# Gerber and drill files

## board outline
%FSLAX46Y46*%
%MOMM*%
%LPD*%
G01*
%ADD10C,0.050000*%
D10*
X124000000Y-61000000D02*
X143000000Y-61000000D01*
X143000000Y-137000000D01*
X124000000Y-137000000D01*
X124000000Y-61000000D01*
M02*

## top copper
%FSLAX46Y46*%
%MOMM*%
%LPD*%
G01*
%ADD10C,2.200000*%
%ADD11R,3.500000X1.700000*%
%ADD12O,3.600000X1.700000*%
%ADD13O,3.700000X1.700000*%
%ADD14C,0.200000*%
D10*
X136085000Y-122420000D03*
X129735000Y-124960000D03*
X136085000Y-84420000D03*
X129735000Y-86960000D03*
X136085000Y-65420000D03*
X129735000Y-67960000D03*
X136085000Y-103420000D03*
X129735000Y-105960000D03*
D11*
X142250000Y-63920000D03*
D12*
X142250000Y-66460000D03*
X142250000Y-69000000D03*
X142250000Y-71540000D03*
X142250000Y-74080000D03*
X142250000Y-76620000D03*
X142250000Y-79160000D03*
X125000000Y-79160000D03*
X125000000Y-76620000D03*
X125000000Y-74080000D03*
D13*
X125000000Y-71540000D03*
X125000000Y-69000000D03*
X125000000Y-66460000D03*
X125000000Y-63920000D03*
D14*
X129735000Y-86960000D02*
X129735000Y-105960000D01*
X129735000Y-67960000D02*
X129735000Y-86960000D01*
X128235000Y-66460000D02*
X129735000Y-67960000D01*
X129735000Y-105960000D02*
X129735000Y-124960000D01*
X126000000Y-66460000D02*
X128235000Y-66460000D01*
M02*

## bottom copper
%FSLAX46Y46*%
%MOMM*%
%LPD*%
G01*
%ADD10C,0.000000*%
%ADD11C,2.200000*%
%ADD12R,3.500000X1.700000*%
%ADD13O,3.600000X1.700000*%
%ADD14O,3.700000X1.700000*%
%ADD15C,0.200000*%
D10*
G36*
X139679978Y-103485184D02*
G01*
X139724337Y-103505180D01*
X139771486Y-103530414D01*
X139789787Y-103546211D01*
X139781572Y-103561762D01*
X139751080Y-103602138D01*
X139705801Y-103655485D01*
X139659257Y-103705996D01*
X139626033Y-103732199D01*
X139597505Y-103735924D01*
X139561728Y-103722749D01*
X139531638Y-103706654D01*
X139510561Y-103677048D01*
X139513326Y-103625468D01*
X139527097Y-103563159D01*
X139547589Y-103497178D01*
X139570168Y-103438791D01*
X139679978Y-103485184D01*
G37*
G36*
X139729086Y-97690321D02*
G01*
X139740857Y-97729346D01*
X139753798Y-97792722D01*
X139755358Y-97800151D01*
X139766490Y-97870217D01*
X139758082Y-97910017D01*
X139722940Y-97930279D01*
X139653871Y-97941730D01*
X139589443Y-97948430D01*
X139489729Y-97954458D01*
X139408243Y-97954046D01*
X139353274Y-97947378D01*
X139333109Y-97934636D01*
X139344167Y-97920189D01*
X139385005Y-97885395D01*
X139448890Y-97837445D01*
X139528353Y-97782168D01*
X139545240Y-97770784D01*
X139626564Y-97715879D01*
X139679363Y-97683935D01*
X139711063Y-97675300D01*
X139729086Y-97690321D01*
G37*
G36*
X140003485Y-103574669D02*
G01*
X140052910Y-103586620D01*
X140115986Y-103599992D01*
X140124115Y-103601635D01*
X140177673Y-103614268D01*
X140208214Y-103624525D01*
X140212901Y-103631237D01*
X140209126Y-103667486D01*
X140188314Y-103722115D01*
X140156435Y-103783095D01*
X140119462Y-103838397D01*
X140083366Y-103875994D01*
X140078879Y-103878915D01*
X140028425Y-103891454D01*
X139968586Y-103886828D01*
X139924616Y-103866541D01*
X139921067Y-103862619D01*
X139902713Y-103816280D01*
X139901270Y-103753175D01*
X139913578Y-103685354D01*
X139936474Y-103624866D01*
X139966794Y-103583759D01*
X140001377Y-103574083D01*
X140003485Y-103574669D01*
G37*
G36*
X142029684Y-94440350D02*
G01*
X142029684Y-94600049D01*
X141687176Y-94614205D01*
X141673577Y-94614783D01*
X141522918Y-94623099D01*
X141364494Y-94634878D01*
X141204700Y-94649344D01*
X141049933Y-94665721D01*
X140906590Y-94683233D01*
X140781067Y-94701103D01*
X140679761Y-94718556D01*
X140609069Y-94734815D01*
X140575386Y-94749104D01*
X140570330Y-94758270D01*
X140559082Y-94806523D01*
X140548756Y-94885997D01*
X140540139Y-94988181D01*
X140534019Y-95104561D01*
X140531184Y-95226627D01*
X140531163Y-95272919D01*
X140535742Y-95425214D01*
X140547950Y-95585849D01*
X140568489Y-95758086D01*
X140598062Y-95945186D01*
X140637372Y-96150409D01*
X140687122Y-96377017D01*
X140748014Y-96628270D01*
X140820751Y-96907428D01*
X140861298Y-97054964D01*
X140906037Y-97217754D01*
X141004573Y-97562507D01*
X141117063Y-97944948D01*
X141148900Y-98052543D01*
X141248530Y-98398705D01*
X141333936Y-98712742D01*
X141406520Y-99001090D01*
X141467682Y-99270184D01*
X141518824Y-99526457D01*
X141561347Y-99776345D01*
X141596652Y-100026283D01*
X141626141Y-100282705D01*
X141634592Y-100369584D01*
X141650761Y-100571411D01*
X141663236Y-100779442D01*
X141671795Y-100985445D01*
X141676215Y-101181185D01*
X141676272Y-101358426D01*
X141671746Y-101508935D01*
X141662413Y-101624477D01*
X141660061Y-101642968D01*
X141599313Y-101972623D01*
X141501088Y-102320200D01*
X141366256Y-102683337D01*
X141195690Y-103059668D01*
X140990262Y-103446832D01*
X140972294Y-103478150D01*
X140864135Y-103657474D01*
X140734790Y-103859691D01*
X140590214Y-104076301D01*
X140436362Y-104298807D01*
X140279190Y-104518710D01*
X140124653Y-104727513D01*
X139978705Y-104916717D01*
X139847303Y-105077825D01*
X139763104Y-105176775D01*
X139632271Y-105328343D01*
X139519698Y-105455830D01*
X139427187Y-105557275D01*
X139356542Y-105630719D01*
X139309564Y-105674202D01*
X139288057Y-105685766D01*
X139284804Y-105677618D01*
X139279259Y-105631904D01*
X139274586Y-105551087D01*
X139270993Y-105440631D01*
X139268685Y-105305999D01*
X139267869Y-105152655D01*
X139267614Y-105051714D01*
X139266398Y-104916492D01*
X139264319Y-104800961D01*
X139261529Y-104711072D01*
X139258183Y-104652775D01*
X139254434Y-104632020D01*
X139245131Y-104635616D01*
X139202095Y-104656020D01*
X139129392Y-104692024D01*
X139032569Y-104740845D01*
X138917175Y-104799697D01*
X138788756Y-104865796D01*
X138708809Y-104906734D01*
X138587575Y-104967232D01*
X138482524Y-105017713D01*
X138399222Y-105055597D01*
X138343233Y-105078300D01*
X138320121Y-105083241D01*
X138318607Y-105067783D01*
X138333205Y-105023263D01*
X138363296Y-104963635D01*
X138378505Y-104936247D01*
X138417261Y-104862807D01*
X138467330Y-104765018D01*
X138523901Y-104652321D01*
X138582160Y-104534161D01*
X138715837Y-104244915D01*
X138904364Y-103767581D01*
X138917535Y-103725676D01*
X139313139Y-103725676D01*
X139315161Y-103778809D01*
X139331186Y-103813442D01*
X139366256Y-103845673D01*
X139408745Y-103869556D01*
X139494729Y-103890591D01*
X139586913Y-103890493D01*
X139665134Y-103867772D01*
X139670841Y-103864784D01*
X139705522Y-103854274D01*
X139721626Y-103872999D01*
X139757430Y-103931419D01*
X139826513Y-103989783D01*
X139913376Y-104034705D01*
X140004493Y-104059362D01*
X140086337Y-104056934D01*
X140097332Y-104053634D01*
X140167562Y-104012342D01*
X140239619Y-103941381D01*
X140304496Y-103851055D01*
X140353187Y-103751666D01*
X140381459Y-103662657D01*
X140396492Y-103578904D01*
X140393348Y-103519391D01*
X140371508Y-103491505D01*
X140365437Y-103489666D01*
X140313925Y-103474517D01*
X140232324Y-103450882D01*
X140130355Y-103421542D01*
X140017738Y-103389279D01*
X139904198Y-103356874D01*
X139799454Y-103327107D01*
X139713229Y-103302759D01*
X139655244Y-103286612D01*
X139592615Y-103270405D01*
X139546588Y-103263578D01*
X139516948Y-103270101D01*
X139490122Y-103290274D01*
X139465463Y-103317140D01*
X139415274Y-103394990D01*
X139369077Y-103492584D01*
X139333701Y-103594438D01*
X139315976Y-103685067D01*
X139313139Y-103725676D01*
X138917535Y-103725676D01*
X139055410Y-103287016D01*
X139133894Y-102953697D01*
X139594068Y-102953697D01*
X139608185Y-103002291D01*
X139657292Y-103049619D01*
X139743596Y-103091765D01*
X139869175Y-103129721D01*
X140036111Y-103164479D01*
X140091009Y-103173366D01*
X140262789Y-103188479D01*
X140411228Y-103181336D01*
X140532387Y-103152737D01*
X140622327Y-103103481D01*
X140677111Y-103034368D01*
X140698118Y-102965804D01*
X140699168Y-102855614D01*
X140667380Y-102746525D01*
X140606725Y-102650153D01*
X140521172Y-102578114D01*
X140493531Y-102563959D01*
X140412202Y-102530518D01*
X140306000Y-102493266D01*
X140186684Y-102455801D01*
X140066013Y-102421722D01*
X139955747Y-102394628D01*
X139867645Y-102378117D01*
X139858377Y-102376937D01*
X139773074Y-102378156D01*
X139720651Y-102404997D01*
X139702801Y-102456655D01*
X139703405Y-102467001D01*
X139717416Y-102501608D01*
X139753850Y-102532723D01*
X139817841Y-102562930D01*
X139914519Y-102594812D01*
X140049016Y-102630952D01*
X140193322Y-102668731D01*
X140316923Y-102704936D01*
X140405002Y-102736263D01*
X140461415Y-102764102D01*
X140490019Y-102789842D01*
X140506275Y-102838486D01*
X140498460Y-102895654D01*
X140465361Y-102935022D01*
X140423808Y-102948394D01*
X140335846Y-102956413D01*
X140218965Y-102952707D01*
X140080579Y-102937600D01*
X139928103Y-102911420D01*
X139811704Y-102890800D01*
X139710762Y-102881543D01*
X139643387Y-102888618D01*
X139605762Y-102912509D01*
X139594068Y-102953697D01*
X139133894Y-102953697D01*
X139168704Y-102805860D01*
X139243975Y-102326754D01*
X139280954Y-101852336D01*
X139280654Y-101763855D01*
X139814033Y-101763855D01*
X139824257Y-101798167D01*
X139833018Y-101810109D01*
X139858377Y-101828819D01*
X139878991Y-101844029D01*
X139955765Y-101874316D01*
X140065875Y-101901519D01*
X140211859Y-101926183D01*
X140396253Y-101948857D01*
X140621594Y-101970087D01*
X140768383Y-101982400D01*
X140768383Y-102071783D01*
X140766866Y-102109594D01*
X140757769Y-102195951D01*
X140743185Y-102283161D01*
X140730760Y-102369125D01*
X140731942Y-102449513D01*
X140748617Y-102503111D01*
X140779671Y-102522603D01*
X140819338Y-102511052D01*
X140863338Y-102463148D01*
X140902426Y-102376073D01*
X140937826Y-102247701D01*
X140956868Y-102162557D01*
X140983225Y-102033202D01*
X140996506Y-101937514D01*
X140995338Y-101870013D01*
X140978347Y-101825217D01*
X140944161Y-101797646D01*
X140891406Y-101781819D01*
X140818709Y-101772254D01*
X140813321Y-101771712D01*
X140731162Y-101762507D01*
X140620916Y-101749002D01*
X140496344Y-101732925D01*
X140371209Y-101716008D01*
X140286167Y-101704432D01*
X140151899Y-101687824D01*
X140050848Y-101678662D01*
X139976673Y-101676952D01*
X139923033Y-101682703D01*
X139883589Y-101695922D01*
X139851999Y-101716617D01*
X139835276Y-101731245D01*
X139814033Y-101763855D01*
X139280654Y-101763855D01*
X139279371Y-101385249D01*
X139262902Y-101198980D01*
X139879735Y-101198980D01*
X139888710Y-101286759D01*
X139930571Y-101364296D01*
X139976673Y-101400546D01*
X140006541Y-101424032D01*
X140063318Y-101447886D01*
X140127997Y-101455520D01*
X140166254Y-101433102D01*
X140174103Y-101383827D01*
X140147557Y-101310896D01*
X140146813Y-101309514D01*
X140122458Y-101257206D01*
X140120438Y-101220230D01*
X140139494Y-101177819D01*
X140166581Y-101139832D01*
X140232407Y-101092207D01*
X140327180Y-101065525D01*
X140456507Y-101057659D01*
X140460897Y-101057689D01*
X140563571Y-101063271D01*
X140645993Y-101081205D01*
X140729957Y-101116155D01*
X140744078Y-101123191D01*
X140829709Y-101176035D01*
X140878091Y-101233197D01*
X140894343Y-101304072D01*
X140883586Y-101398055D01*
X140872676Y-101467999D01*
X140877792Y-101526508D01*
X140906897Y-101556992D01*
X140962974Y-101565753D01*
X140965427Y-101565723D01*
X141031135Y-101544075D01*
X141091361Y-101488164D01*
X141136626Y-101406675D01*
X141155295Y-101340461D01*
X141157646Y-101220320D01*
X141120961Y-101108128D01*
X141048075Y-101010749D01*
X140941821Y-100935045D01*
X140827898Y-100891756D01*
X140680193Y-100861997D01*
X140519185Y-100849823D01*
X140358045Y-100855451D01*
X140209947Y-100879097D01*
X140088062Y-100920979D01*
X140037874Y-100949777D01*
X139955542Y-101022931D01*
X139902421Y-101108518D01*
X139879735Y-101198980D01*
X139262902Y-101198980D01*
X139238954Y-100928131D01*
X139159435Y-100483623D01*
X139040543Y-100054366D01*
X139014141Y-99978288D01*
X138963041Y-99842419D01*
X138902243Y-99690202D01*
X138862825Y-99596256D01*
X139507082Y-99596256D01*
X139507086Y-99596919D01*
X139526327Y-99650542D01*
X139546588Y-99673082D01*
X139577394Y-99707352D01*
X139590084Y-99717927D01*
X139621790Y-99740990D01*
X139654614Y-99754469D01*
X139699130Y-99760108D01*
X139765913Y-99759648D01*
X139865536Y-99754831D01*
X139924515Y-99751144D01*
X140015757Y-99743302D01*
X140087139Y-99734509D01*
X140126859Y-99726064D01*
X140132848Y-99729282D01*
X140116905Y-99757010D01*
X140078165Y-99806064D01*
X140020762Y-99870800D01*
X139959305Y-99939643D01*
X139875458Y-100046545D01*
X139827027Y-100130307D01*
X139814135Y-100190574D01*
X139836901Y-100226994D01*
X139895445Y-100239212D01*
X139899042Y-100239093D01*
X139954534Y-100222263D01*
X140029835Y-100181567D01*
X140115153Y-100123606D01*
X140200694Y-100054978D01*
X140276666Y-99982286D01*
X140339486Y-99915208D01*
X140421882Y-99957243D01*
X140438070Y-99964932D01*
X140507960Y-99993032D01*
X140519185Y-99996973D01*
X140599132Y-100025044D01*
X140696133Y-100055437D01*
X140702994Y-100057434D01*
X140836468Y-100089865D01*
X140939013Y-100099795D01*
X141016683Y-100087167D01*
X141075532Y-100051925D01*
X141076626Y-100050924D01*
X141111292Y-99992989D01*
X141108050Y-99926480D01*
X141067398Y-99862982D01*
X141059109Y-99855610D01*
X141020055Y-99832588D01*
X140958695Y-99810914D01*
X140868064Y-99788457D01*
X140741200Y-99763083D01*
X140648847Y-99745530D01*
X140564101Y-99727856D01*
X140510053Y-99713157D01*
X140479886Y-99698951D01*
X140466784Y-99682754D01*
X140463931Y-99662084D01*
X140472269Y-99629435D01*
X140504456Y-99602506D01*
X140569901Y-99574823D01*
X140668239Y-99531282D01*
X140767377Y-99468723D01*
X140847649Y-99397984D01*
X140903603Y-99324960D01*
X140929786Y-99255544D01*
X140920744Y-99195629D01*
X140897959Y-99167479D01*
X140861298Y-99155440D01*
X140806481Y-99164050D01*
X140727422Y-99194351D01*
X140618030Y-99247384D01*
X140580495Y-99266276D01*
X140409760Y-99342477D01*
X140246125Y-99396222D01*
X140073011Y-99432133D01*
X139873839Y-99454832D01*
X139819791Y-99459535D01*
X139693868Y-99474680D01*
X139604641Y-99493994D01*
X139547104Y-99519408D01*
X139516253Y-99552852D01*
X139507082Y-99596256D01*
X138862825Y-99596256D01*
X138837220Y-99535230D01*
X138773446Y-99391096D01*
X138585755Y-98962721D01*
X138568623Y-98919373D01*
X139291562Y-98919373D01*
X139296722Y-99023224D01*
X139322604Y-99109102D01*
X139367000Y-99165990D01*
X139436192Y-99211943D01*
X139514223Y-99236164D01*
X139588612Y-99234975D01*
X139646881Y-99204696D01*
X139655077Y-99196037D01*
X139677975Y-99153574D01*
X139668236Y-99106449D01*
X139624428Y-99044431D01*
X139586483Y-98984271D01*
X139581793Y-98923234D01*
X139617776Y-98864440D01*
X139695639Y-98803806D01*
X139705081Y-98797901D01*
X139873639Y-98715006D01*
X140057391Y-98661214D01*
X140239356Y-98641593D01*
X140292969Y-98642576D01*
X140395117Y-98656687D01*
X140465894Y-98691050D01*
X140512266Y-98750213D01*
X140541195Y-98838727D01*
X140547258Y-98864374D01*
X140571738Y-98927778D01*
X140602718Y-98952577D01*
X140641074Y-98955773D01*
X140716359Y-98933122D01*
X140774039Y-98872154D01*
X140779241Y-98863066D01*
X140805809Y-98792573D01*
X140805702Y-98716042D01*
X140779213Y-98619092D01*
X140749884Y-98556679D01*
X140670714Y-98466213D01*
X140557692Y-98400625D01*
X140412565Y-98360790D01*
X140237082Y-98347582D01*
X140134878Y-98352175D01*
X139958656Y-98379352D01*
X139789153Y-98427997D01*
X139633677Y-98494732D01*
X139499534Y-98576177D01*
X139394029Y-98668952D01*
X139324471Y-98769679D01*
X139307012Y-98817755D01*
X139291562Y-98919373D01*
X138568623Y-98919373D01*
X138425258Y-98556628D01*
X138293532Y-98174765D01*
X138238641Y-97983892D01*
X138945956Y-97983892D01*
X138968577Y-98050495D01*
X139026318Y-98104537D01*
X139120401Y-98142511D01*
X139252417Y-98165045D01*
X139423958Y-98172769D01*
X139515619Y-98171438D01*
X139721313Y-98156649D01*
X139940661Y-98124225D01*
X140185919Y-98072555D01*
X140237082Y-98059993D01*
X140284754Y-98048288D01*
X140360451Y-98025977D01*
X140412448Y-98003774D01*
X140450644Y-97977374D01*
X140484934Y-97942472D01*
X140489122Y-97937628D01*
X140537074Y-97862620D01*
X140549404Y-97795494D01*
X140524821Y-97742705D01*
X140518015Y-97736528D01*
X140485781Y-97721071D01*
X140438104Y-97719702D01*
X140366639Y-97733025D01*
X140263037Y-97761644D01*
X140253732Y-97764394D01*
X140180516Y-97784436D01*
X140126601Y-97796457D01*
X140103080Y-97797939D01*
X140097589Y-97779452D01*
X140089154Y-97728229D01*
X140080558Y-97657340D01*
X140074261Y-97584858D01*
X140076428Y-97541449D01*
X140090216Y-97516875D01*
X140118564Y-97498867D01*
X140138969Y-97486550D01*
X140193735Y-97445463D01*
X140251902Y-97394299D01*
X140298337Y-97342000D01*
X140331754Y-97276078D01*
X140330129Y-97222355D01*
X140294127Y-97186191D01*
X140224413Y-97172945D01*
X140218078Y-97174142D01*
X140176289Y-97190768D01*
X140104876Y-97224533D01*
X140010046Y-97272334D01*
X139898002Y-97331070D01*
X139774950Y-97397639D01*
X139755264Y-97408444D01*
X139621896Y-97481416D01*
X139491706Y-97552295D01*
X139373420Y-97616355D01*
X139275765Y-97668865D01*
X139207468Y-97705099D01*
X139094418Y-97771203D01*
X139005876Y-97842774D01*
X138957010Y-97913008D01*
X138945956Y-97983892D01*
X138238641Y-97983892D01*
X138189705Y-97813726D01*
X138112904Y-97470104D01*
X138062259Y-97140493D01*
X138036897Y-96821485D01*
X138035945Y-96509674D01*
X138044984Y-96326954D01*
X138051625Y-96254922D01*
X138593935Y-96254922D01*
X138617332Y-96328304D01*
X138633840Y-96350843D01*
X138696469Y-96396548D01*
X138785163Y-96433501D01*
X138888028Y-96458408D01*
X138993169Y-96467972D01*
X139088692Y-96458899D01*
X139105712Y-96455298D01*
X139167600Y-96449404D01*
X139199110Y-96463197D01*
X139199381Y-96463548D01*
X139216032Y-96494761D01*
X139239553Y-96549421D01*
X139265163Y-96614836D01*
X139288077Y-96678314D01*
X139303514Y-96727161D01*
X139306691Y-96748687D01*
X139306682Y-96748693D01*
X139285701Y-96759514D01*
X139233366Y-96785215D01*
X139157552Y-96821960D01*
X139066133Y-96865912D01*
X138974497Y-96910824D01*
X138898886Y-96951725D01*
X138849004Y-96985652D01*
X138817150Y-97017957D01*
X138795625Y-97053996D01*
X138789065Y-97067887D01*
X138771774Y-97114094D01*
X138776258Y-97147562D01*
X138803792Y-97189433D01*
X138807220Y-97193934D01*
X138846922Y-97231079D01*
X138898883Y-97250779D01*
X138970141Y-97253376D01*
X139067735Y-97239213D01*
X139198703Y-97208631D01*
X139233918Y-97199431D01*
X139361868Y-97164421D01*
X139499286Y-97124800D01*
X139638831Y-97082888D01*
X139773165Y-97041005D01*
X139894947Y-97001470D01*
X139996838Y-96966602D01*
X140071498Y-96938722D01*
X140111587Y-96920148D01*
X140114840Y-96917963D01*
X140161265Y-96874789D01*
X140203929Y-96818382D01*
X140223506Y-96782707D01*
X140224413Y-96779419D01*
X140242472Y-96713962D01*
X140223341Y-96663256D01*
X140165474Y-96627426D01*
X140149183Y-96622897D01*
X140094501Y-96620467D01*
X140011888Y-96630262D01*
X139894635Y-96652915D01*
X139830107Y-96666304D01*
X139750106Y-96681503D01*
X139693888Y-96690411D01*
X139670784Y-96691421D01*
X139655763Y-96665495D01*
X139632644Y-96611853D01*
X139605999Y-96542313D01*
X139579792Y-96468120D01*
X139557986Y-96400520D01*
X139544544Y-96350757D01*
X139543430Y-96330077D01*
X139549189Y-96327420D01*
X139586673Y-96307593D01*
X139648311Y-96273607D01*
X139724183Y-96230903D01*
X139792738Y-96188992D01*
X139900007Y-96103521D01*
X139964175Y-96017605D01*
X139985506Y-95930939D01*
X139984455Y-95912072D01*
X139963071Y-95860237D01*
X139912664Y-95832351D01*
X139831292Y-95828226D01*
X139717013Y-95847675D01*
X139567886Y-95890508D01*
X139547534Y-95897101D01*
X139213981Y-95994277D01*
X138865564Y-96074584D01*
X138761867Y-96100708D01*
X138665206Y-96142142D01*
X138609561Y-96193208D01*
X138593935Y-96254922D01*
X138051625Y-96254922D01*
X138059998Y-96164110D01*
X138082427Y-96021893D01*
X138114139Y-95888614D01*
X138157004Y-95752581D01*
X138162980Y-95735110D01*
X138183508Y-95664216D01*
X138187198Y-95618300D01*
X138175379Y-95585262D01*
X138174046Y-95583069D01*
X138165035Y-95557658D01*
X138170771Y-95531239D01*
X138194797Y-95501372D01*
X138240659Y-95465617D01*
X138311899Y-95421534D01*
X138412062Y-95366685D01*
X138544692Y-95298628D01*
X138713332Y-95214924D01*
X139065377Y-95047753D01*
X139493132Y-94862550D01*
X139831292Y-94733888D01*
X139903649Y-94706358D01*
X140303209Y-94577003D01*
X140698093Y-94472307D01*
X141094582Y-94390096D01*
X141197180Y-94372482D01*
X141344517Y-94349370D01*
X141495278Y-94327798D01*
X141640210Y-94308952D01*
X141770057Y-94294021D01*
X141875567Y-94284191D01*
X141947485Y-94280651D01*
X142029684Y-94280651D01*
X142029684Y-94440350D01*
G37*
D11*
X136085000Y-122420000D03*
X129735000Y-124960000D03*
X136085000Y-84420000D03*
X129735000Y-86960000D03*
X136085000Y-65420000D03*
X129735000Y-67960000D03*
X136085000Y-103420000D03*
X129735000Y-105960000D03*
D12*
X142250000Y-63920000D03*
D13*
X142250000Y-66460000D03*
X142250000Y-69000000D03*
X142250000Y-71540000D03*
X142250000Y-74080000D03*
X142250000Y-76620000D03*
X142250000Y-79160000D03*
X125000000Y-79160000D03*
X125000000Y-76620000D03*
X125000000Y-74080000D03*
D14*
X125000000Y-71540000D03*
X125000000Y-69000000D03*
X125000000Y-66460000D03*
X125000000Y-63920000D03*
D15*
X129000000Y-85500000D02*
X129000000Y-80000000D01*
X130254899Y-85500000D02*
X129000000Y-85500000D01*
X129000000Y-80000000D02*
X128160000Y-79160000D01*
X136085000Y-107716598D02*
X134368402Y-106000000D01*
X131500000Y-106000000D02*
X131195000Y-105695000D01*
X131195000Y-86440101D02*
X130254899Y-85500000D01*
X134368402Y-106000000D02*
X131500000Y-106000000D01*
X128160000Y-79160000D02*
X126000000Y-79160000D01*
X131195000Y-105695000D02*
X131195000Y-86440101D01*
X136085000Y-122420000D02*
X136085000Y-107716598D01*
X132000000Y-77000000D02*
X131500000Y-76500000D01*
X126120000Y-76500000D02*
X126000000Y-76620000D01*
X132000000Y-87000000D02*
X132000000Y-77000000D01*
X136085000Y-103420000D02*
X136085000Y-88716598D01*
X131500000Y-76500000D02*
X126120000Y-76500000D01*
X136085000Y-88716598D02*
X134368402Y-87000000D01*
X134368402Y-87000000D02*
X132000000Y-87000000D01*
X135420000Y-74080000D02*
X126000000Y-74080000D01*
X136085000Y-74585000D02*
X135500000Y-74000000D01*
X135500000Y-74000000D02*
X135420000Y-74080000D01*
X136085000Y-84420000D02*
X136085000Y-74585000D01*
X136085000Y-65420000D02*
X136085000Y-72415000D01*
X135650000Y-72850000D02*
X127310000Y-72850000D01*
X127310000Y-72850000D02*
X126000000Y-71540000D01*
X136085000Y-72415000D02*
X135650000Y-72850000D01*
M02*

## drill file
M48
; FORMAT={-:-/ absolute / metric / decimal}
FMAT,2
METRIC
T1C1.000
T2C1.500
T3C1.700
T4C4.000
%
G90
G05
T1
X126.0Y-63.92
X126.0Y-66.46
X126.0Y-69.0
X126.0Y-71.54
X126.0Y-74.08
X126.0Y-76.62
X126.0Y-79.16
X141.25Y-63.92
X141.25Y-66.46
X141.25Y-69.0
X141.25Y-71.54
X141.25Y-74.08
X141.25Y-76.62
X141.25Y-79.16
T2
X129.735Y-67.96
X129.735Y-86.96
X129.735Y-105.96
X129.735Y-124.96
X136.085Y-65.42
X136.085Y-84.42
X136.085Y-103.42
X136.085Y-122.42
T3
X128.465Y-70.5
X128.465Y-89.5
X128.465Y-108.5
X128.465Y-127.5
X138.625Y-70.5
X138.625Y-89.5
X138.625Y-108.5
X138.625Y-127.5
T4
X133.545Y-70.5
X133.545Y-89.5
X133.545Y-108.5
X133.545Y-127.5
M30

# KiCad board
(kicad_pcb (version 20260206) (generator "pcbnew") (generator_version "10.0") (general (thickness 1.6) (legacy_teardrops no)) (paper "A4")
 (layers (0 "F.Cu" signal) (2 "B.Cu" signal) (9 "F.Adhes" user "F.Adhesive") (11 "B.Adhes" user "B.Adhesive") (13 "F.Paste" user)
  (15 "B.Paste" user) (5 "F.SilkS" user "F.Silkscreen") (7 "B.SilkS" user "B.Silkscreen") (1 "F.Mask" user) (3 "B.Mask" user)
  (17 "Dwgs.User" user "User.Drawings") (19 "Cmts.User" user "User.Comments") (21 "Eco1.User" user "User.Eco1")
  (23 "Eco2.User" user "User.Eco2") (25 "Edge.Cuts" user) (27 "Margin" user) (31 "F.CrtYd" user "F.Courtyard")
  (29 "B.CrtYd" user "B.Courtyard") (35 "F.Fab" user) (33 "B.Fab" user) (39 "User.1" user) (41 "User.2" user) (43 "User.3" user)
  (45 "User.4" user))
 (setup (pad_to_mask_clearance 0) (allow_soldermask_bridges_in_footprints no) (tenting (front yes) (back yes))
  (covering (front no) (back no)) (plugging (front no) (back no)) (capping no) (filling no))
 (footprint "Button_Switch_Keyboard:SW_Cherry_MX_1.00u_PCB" (layer "F.Cu") (at 136.085 122.42)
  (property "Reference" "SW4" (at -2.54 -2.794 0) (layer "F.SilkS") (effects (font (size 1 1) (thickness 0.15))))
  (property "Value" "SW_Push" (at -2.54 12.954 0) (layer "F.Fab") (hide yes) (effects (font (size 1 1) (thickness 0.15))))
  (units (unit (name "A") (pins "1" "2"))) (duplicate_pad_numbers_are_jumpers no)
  (pad "" np_thru_hole circle (at -7.62 5.08) (size 1.7 1.7) (drill 1.7) (layers "*.Cu" "*.Mask"))
  (pad "" np_thru_hole circle (at -2.54 5.08) (size 4 4) (drill 4) (layers "*.Cu" "*.Mask"))
  (pad "" np_thru_hole circle (at 2.54 5.08) (size 1.7 1.7) (drill 1.7) (layers "*.Cu" "*.Mask"))
  (pad "1" thru_hole circle (at 0 0) (size 2.2 2.2) (drill 1.5) (layers "*.Cu" "*.Mask") (remove_unused_layers no)
   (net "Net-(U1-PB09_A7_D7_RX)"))
  (pad "2" thru_hole circle (at -6.35 2.54) (size 2.2 2.2) (drill 1.5) (layers "*.Cu" "*.Mask") (remove_unused_layers no) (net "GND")))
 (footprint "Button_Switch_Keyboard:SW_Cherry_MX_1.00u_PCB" (layer "F.Cu") (at 136.085 84.42)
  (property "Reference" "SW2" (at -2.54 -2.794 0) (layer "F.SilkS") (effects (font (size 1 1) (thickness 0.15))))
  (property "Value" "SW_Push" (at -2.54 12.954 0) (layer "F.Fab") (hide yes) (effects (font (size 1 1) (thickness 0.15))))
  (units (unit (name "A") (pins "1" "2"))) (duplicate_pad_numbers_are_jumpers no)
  (pad "" np_thru_hole circle (at -7.62 5.08) (size 1.7 1.7) (drill 1.7) (layers "*.Cu" "*.Mask"))
  (pad "" np_thru_hole circle (at -2.54 5.08) (size 4 4) (drill 4) (layers "*.Cu" "*.Mask"))
  (pad "" np_thru_hole circle (at 2.54 5.08) (size 1.7 1.7) (drill 1.7) (layers "*.Cu" "*.Mask"))
  (pad "1" thru_hole circle (at 0 0) (size 2.2 2.2) (drill 1.5) (layers "*.Cu" "*.Mask") (remove_unused_layers no)
   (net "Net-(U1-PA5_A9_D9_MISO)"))
  (pad "2" thru_hole circle (at -6.35 2.54) (size 2.2 2.2) (drill 1.5) (layers "*.Cu" "*.Mask") (remove_unused_layers no) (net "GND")))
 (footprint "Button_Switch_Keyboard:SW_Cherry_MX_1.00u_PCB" (layer "F.Cu") (at 136.085 65.42)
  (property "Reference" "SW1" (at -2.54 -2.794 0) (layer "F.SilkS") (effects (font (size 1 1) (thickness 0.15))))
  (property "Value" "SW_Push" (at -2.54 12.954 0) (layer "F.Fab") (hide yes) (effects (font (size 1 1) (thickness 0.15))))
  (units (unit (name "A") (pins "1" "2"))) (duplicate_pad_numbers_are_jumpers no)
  (pad "" np_thru_hole circle (at -7.62 5.08) (size 1.7 1.7) (drill 1.7) (layers "*.Cu" "*.Mask"))
  (pad "" np_thru_hole circle (at -2.54 5.08) (size 4 4) (drill 4) (layers "*.Cu" "*.Mask"))
  (pad "" np_thru_hole circle (at 2.54 5.08) (size 1.7 1.7) (drill 1.7) (layers "*.Cu" "*.Mask"))
  (pad "1" thru_hole circle (at 0 0) (size 2.2 2.2) (drill 1.5) (layers "*.Cu" "*.Mask") (remove_unused_layers no)
   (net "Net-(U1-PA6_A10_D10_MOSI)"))
  (pad "2" thru_hole circle (at -6.35 2.54) (size 2.2 2.2) (drill 1.5) (layers "*.Cu" "*.Mask") (remove_unused_layers no) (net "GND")))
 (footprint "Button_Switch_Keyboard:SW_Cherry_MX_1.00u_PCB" (layer "F.Cu") (at 136.085 103.42)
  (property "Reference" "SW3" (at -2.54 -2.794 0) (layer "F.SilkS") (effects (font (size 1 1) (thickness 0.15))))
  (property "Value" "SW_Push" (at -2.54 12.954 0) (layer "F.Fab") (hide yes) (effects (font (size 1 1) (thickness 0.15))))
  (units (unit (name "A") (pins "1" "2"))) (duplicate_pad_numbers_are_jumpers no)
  (pad "" np_thru_hole circle (at -7.62 5.08) (size 1.7 1.7) (drill 1.7) (layers "*.Cu" "*.Mask"))
  (pad "" np_thru_hole circle (at -2.54 5.08) (size 4 4) (drill 4) (layers "*.Cu" "*.Mask"))
  (pad "" np_thru_hole circle (at 2.54 5.08) (size 1.7 1.7) (drill 1.7) (layers "*.Cu" "*.Mask"))
  (pad "1" thru_hole circle (at 0 0) (size 2.2 2.2) (drill 1.5) (layers "*.Cu" "*.Mask") (remove_unused_layers no)
   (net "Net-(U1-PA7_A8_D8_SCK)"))
  (pad "2" thru_hole circle (at -6.35 2.54) (size 2.2 2.2) (drill 1.5) (layers "*.Cu" "*.Mask") (remove_unused_layers no) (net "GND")))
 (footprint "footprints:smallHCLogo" (layer "B.Cu") (at 140.029 100 -90)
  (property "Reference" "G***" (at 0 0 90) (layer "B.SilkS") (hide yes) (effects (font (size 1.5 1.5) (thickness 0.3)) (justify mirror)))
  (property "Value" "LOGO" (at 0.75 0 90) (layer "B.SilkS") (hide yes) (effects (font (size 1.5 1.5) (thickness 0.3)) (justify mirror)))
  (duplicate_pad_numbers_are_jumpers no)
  (fp_poly
   (pts (xy 3.706654 0.497362) (xy 3.722749 0.467272) (xy 3.735924 0.431495) (xy 3.732199 0.402967) (xy 3.705996 0.369743)
    (xy 3.655485 0.323199) (xy 3.602138 0.27792) (xy 3.561762 0.247428) (xy 3.546211 0.239213) (xy 3.530414 0.257514) (xy 3.50518 0.304663)
    (xy 3.485184 0.349022) (xy 3.438791 0.458832) (xy 3.497178 0.481411) (xy 3.563159 0.501903) (xy 3.625468 0.515674)
    (xy 3.677048 0.518439))
   (stroke (width 0) (type solid)) (fill yes) (layer "B.Cu"))
  (fp_poly
   (pts (xy -2.052622 0.675726) (xy -2.045954 0.620757) (xy -2.045542 0.539271) (xy -2.05157 0.439557) (xy -2.05827 0.375129)
    (xy -2.069721 0.30606) (xy -2.089983 0.270918) (xy -2.129783 0.26251) (xy -2.199849 0.273642) (xy -2.207278 0.275202)
    (xy -2.270654 0.288143) (xy -2.309679 0.299914) (xy -2.3247 0.317937) (xy -2.316065 0.349637) (xy -2.284121 0.402436)
    (xy -2.229216 0.48376) (xy -2.217832 0.500647) (xy -2.162555 0.58011) (xy -2.114605 0.643995) (xy -2.079811 0.684833)
    (xy -2.065364 0.695891))
   (stroke (width 0) (type solid)) (fill yes) (layer "B.Cu"))
  (fp_poly
   (pts (xy 3.81628 0.126287) (xy 3.862619 0.107933) (xy 3.866541 0.104384) (xy 3.886828 0.060414) (xy 3.891454 0.000575)
    (xy 3.878915 -0.049879) (xy 3.875994 -0.054366) (xy 3.838397 -0.090462) (xy 3.783095 -0.127435) (xy 3.722115 -0.159314)
    (xy 3.667486 -0.180126) (xy 3.631237 -0.183901) (xy 3.624525 -0.179214) (xy 3.614268 -0.148673) (xy 3.601635 -0.095115)
    (xy 3.599992 -0.086986) (xy 3.58662 -0.02391) (xy 3.574669 0.025515) (xy 3.574083 0.027623) (xy 3.583759 0.062206)
    (xy 3.624866 0.092526) (xy 3.685354 0.115422) (xy 3.753175 0.12773))
   (stroke (width 0) (type solid)) (fill yes) (layer "B.Cu"))
  (fp_poly
   (pts (xy -3.178515 1.992103) (xy -2.859507 1.966741) (xy -2.529896 1.916096) (xy -2.186274 1.839295) (xy -1.825235 1.735468)
    (xy -1.443372 1.603742) (xy -1.037279 1.443245) (xy -0.608904 1.255554) (xy -0.46477 1.19178) (xy -0.309798 1.126757)
    (xy -0.157581 1.065959) (xy -0.021712 1.014859) (xy 0.054366 0.988457) (xy 0.483623 0.869565) (xy 0.928131 0.790046)
    (xy 1.385249 0.749629) (xy 1.852336 0.748046) (xy 2.326754 0.785025) (xy 2.80586 0.860296) (xy 3.287016 0.97359) (xy 3.767581 1.124636)
    (xy 4.244915 1.313163) (xy 4.534161 1.44684) (xy 4.652321 1.505099) (xy 4.765018 1.56167) (xy 4.862807 1.611739) (xy 4.936247 1.650495)
    (xy 4.963635 1.665704) (xy 5.023263 1.695795) (xy 5.067783 1.710393) (xy 5.083241 1.708879) (xy 5.0783 1.685767) (xy 5.055597 1.629778)
    (xy 5.017713 1.546476) (xy 4.967232 1.441425) (xy 4.906734 1.320191) (xy 4.865796 1.240244) (xy 4.799697 1.111825)
    (xy 4.740845 0.996431) (xy 4.692024 0.899608) (xy 4.65602 0.826905) (xy 4.635616 0.783869) (xy 4.63202 0.774566) (xy 4.652775 0.770817)
    (xy 4.711072 0.767471) (xy 4.800961 0.764681) (xy 4.916492 0.762602) (xy 5.051714 0.761386) (xy 5.152655 0.761131)
    (xy 5.305999 0.760315) (xy 5.440631 0.758007) (xy 5.551087 0.754414) (xy 5.631904 0.749741) (xy 5.677618 0.744196)
    (xy 5.685766 0.740943) (xy 5.674202 0.719436) (xy 5.630719 0.672458) (xy 5.557275 0.601813) (xy 5.45583 0.509302) (xy 5.328343 0.396729)
    (xy 5.176775 0.265896) (xy 5.077825 0.181697) (xy 4.916717 0.050295) (xy 4.727513 -0.095653) (xy 4.51871 -0.25019)
    (xy 4.298807 -0.407362) (xy 4.076301 -0.561214) (xy 3.859691 -0.70579) (xy 3.657474 -0.835135) (xy 3.47815 -0.943294)
    (xy 3.446832 -0.961262) (xy 3.059668 -1.16669) (xy 2.683337 -1.337256) (xy 2.3202 -1.472088) (xy 1.972623 -1.570313)
    (xy 1.642968 -1.631061) (xy 1.624477 -1.633413) (xy 1.508935 -1.642746) (xy 1.358426 -1.647272) (xy 1.181185 -1.647215)
    (xy 0.985445 -1.642795) (xy 0.779442 -1.634236) (xy 0.571411 -1.621761) (xy 0.369584 -1.605592) (xy 0.282705 -1.597141)
    (xy 0.026283 -1.567652) (xy -0.223655 -1.532347) (xy -0.473543 -1.489824) (xy -0.729816 -1.438682) (xy -0.99891 -1.37752)
    (xy -1.287258 -1.304936) (xy -1.601295 -1.21953) (xy -1.947457 -1.1199) (xy -2.055052 -1.088063) (xy -2.437493 -0.975573)
    (xy -2.782246 -0.877037) (xy -2.945036 -0.832298) (xy -0.84456 -0.832298) (xy -0.832521 -0.868959) (xy -0.804371 -0.891744)
    (xy -0.744456 -0.900786) (xy -0.67504 -0.874603) (xy -0.602016 -0.818649) (xy -0.531277 -0.738377) (xy -0.468718 -0.639239)
    (xy -0.425177 -0.540901) (xy -0.397494 -0.475456) (xy -0.370565 -0.443269) (xy -0.337916 -0.434931) (xy -0.317246 -0.437784)
    (xy -0.301049 -0.450886) (xy -0.286843 -0.481053) (xy -0.272144 -0.535101) (xy -0.25447 -0.619847) (xy -0.236917 -0.7122)
    (xy -0.211543 -0.839064) (xy -0.189086 -0.929695) (xy -0.167412 -0.991055) (xy -0.14439 -1.030109) (xy -0.137018 -1.038398)
    (xy -0.07352 -1.07905) (xy -0.007011 -1.082292) (xy 0.050924 -1.047626) (xy 0.051925 -1.046532) (xy 0.087167 -0.987683)
    (xy 0.099795 -0.910013) (xy 0.089865 -0.807468) (xy 0.057434 -0.673994) (xy 0.055437 -0.667133) (xy 0.025044 -0.570132)
    (xy -0.003027 -0.490185) (xy 0.849823 -0.490185) (xy 0.861997 -0.651193) (xy 0.891756 -0.798898) (xy 0.935045 -0.912821)
    (xy 1.010749 -1.019075) (xy 1.108128 -1.091961) (xy 1.22032 -1.128646) (xy 1.340461 -1.126295) (xy 1.406675 -1.107626)
    (xy 1.488164 -1.062361) (xy 1.544075 -1.002135) (xy 1.565723 -0.936427) (xy 1.565753 -0.933974) (xy 1.556992 -0.877897)
    (xy 1.526508 -0.848792) (xy 1.467999 -0.843676) (xy 1.398055 -0.854586) (xy 1.304072 -0.865343) (xy 1.233197 -0.849091)
    (xy 1.176035 -0.800709) (xy 1.123191 -0.715078) (xy 1.116155 -0.700957) (xy 1.081205 -0.616993) (xy 1.063271 -0.534571)
    (xy 1.057689 -0.431897) (xy 1.057659 -0.427507) (xy 1.065525 -0.29818) (xy 1.092207 -0.203407) (xy 1.139832 -0.137581)
    (xy 1.177819 -0.110494) (xy 1.22023 -0.091438) (xy 1.257206 -0.093458) (xy 1.309514 -0.117813) (xy 1.310896 -0.118557)
    (xy 1.383827 -0.145103) (xy 1.433102 -0.137254) (xy 1.45552 -0.098997) (xy 1.447886 -0.034318) (xy 1.424032 0.022459)
    (xy 1.400546 0.052327) (xy 1.676952 0.052327) (xy 1.678662 -0.021848) (xy 1.687824 -0.122899) (xy 1.704432 -0.257167)
    (xy 1.716008 -0.342209) (xy 1.732925 -0.467344) (xy 1.749002 -0.591916) (xy 1.762507 -0.702162) (xy 1.771712 -0.784321)
    (xy 1.772254 -0.789709) (xy 1.781819 -0.862406) (xy 1.797646 -0.915161) (xy 1.825217 -0.949347) (xy 1.870013 -0.966338)
    (xy 1.937514 -0.967506) (xy 2.033202 -0.954225) (xy 2.162557 -0.927868) (xy 2.247701 -0.908826) (xy 2.376073 -0.873426)
    (xy 2.463148 -0.834338) (xy 2.511052 -0.790338) (xy 2.522603 -0.750671) (xy 2.503111 -0.719617) (xy 2.449513 -0.702942)
    (xy 2.369125 -0.70176) (xy 2.283161 -0.714185) (xy 2.195951 -0.728769) (xy 2.109594 -0.737866) (xy 2.071783 -0.739383)
    (xy 1.9824 -0.739383) (xy 1.970087 -0.592594) (xy 1.948857 -0.367253) (xy 1.926183 -0.182859) (xy 1.901519 -0.036875)
    (xy 1.874316 0.073235) (xy 1.844029 0.150009) (xy 1.828819 0.170623) (xy 2.376937 0.170623) (xy 2.378117 0.161355)
    (xy 2.394628 0.073253) (xy 2.421722 -0.037013) (xy 2.455801 -0.157684) (xy 2.493266 -0.277) (xy 2.530518 -0.383202)
    (xy 2.563959 -0.464531) (xy 2.578114 -0.492172) (xy 2.650153 -0.577725) (xy 2.746525 -0.63838) (xy 2.855614 -0.670168)
    (xy 2.965804 -0.669118) (xy 3.034368 -0.648111) (xy 3.103481 -0.593327) (xy 3.152737 -0.503387) (xy 3.181336 -0.382228)
    (xy 3.188479 -0.233789) (xy 3.173366 -0.062009) (xy 3.164479 -0.007111) (xy 3.129721 0.159825) (xy 3.091765 0.285404)
    (xy 3.049619 0.371708) (xy 3.002291 0.420815) (xy 2.953697 0.434932) (xy 2.912509 0.423238) (xy 2.888618 0.385613)
    (xy 2.881543 0.318238) (xy 2.8908 0.217296) (xy 2.91142 0.100897) (xy 2.9376 -0.051579) (xy 2.952707 -0.189965) (xy 2.956413 -0.306846)
    (xy 2.948394 -0.394808) (xy 2.935022 -0.436361) (xy 2.895654 -0.46946) (xy 2.838486 -0.477275) (xy 2.789842 -0.461019)
    (xy 2.764102 -0.432415) (xy 2.736263 -0.376002) (xy 2.704936 -0.287923) (xy 2.668731 -0.164322) (xy 2.630952 -0.020016)
    (xy 2.594812 0.114481) (xy 2.56293 0.211159) (xy 2.532723 0.27515) (xy 2.501608 0.311584) (xy 2.467001 0.325595) (xy 2.456655 0.326199)
    (xy 2.404997 0.308349) (xy 2.378156 0.255926) (xy 2.376937 0.170623) (xy 1.828819 0.170623) (xy 1.810109 0.195982)
    (xy 1.798167 0.204743) (xy 1.763855 0.214967) (xy 1.731245 0.193724) (xy 1.716617 0.177001) (xy 1.695922 0.145411)
    (xy 1.682703 0.105967) (xy 1.676952 0.052327) (xy 1.400546 0.052327) (xy 1.364296 0.098429) (xy 1.286759 0.14029) (xy 1.19898 0.149265)
    (xy 1.108518 0.126579) (xy 1.022931 0.073458) (xy 0.949777 -0.008874) (xy 0.920979 -0.059062) (xy 0.879097 -0.180947)
    (xy 0.855451 -0.329045) (xy 0.849823 -0.490185) (xy -0.003027 -0.490185) (xy -0.006968 -0.47896) (xy -0.035068 -0.40907)
    (xy -0.042757 -0.392882) (xy -0.084792 -0.310486) (xy -0.017714 -0.247666) (xy 0.054978 -0.171694) (xy 0.123606 -0.086153)
    (xy 0.181567 -0.000835) (xy 0.222263 0.074466) (xy 0.239093 0.129958) (xy 0.239212 0.133555) (xy 0.226994 0.192099)
    (xy 0.190574 0.214865) (xy 0.130307 0.201973) (xy 0.046545 0.153542) (xy -0.060357 0.069695) (xy -0.1292 0.008238)
    (xy -0.193936 -0.049165) (xy -0.24299 -0.087905) (xy -0.270718 -0.103848) (xy -0.273936 -0.097859) (xy -0.265491 -0.058139)
    (xy -0.256698 0.013243) (xy -0.248856 0.104485) (xy -0.245169 0.163464) (xy -0.240352 0.263087) (xy -0.239892 0.32987)
    (xy -0.245531 0.374386) (xy -0.25901 0.40721) (xy -0.282073 0.438916) (xy -0.292648 0.451606) (xy -0.326918 0.482412)
    (xy 3.263578 0.482412) (xy 3.270405 0.436385) (xy 3.286612 0.373756) (xy 3.302759 0.315771) (xy 3.327107 0.229546)
    (xy 3.356874 0.124802) (xy 3.389279 0.011262) (xy 3.421542 -0.101355) (xy 3.450882 -0.203324) (xy 3.474517 -0.284925)
    (xy 3.489666 -0.336437) (xy 3.491505 -0.342508) (xy 3.519391 -0.364348) (xy 3.578904 -0.367492) (xy 3.662657 -0.352459)
    (xy 3.751666 -0.324187) (xy 3.851055 -0.275496) (xy 3.941381 -0.210619) (xy 4.012342 -0.138562) (xy 4.053634 -0.068332)
    (xy 4.056934 -0.057337) (xy 4.059362 0.024507) (xy 4.034705 0.115624) (xy 3.989783 0.202487) (xy 3.931419 0.27157)
    (xy 3.872999 0.307374) (xy 3.854274 0.323478) (xy 3.864784 0.358159) (xy 3.867772 0.363866) (xy 3.890493 0.442087)
    (xy 3.890591 0.534271) (xy 3.869556 0.620255) (xy 3.845673 0.662744) (xy 3.813442 0.697814) (xy 3.778809 0.713839)
    (xy 3.725676 0.715861) (xy 3.685067 0.713024) (xy 3.594438 0.695299) (xy 3.492584 0.659923) (xy 3.39499 0.613726) (xy 3.31714 0.563537)
    (xy 3.290274 0.538878) (xy 3.270101 0.512052) (xy 3.263578 0.482412) (xy -0.326918 0.482412) (xy -0.349458 0.502673)
    (xy -0.403081 0.521914) (xy -0.403744 0.521918) (xy -0.447148 0.512747) (xy -0.480592 0.481896) (xy -0.506006 0.424359)
    (xy -0.52532 0.335132) (xy -0.540465 0.209209) (xy -0.545168 0.155161) (xy -0.567867 -0.044011) (xy -0.603778 -0.217125)
    (xy -0.657523 -0.38076) (xy -0.733724 -0.551495) (xy -0.752616 -0.58903) (xy -0.805649 -0.698422) (xy -0.83595 -0.777481)
    (xy -0.84456 -0.832298) (xy -2.945036 -0.832298) (xy -3.092572 -0.791751) (xy -3.37173 -0.719014) (xy -3.622983 -0.658122)
    (xy -3.849591 -0.608372) (xy -4.054814 -0.569062) (xy -4.241914 -0.539489) (xy -4.414151 -0.51895) (xy -4.574786 -0.506742)
    (xy -4.727081 -0.502163) (xy -4.773373 -0.502184) (xy -4.895439 -0.505019) (xy -5.011819 -0.511139) (xy -5.114003 -0.519756)
    (xy -5.193477 -0.530082) (xy -5.24173 -0.54133) (xy -5.250896 -0.546386) (xy -5.265185 -0.580069) (xy -5.281444 -0.650761)
    (xy -5.298897 -0.752067) (xy -5.316767 -0.87759) (xy -5.334279 -1.020933) (xy -5.350656 -1.1757) (xy -5.365122 -1.335494)
    (xy -5.376901 -1.493918) (xy -5.385217 -1.644577) (xy -5.385795 -1.658176) (xy -5.399951 -2.000684) (xy -5.55965 -2.000684)
    (xy -5.719349 -2.000684) (xy -5.719349 -1.918485) (xy -5.715809 -1.846567) (xy -5.705979 -1.741057) (xy -5.691048 -1.61121)
    (xy -5.672202 -1.466278) (xy -5.65063 -1.315517) (xy -5.627518 -1.16818) (xy -5.609904 -1.065582) (xy -5.527693 -0.669093)
    (xy -5.422997 -0.274209) (xy -5.293642 0.125351) (xy -5.266112 0.197708) (xy -4.171774 0.197708) (xy -4.167649 0.116336)
    (xy -4.139763 0.065929) (xy -4.087928 0.044545) (xy -4.069061 0.043494) (xy -3.982395 0.064825) (xy -3.896479 0.128993)
    (xy -3.811008 0.236262) (xy -3.769097 0.304817) (xy -3.726393 0.380689) (xy -3.692407 0.442327) (xy -3.67258 0.479811)
    (xy -3.669923 0.48557) (xy -3.649243 0.484456) (xy -3.59948 0.471014) (xy -3.53188 0.449208) (xy -3.457687 0.423001)
    (xy -3.388147 0.396356) (xy -3.334505 0.373237) (xy -3.308579 0.358216) (xy -3.309589 0.335112) (xy -3.318497 0.278894)
    (xy -3.333696 0.198893) (xy -3.347085 0.134365) (xy -3.369738 0.017112) (xy -3.379533 -0.065501) (xy -3.377103 -0.120183)
    (xy -3.372574 -0.136474) (xy -3.336744 -0.194341) (xy -3.286038 -0.213472) (xy -3.220581 -0.195413) (xy -2.827055 -0.195413)
    (xy -2.813809 -0.265127) (xy -2.777645 -0.301129) (xy -2.723922 -0.302754) (xy -2.658 -0.269337) (xy -2.605701 -0.222902)
    (xy -2.554537 -0.164735) (xy -2.51345 -0.109969) (xy -2.501133 -0.089564) (xy -2.483125 -0.061216) (xy -2.458551 -0.047428)
    (xy -2.415142 -0.045261) (xy -2.34266 -0.051558) (xy -2.271771 -0.060154) (xy -2.220548 -0.068589) (xy -2.202061 -0.07408)
    (xy -2.203543 -0.097601) (xy -2.215564 -0.151516) (xy -2.235606 -0.224732) (xy -2.238356 -0.234037) (xy -2.266975 -0.337639)
    (xy -2.280298 -0.409104) (xy -2.278929 -0.456781) (xy -2.263472 -0.489015) (xy -2.257295 -0.495821) (xy -2.204506 -0.520404)
    (xy -2.13738 -0.508074) (xy -2.062372 -0.460122) (xy -2.057528 -0.455934) (xy -2.022626 -0.421644) (xy -1.996226 -0.383448)
    (xy -1.974023 -0.331451) (xy -1.951712 -0.255754) (xy -1.940007 -0.208082) (xy -1.652418 -0.208082) (xy -1.63921 -0.383565)
    (xy -1.599375 -0.528692) (xy -1.533787 -0.641714) (xy -1.443321 -0.720884) (xy -1.380908 -0.750213) (xy -1.283958 -0.776702)
    (xy -1.207427 -0.776809) (xy -1.136934 -0.750241) (xy -1.127846 -0.745039) (xy -1.066878 -0.687359) (xy -1.044227 -0.612074)
    (xy -1.047423 -0.573718) (xy -1.072222 -0.542738) (xy -1.135626 -0.518258) (xy -1.161273 -0.512195) (xy -1.249787 -0.483266)
    (xy -1.30895 -0.436894) (xy -1.343313 -0.366117) (xy -1.357424 -0.263969) (xy -1.358407 -0.210356) (xy -1.338786 -0.028391)
    (xy -1.284994 0.155361) (xy -1.202099 0.323919) (xy -1.196194 0.333361) (xy -1.13556 0.411224) (xy -1.076766 0.447207)
    (xy -1.015729 0.442517) (xy -0.955569 0.404572) (xy -0.893551 0.360764) (xy -0.846426 0.351025) (xy -0.803963 0.373923)
    (xy -0.795304 0.382119) (xy -0.765025 0.440388) (xy -0.763836 0.514777) (xy -0.788057 0.592808) (xy -0.83401 0.662)
    (xy -0.890898 0.706396) (xy -0.976776 0.732278) (xy -1.080627 0.737438) (xy -1.182245 0.721988) (xy -1.230321 0.704529)
    (xy -1.331048 0.634971) (xy -1.423823 0.529466) (xy -1.505268 0.395323) (xy -1.572003 0.239847) (xy -1.620648 0.070344)
    (xy -1.647825 -0.105878) (xy -1.652418 -0.208082) (xy -1.940007 -0.208082) (xy -1.927445 -0.156919) (xy -1.875775 0.088339)
    (xy -1.843351 0.307687) (xy -1.828562 0.513381) (xy -1.827231 0.605042) (xy -1.834955 0.776583) (xy -1.857489 0.908599)
    (xy -1.895463 1.002682) (xy -1.949505 1.060423) (xy -2.016108 1.083044) (xy -2.086992 1.07199) (xy -2.157226 1.023124)
    (xy -2.228797 0.934582) (xy -2.294901 0.821532) (xy -2.331135 0.753235) (xy -2.383645 0.65558) (xy -2.447705 0.537294)
    (xy -2.518584 0.407104) (xy -2.591556 0.273736) (xy -2.602361 0.25405) (xy -2.66893 0.130998) (xy -2.727666 0.018954)
    (xy -2.775467 -0.075876) (xy -2.809232 -0.147289) (xy -2.825858 -0.189078) (xy -2.827055 -0.195413) (xy -3.220581 -0.195413)
    (xy -3.217293 -0.194506) (xy -3.181618 -0.174929) (xy -3.125211 -0.132265) (xy -3.082037 -0.08584) (xy -3.079852 -0.082587)
    (xy -3.061278 -0.042498) (xy -3.033398 0.032162) (xy -2.99853 0.134053) (xy -2.958995 0.255835) (xy -2.917112 0.390169)
    (xy -2.8752 0.529714) (xy -2.835579 0.667132) (xy -2.800569 0.795082) (xy -2.791369 0.830297) (xy -2.760787 0.961265)
    (xy -2.746624 1.058859) (xy -2.749221 1.130117) (xy -2.768921 1.182078) (xy -2.806066 1.22178) (xy -2.810567 1.225208)
    (xy -2.852438 1.252742) (xy -2.885906 1.257226) (xy -2.932113 1.239935) (xy -2.946004 1.233375) (xy -2.982043 1.21185)
    (xy -3.014348 1.179996) (xy -3.048275 1.130114) (xy -3.089176 1.054503) (xy -3.134088 0.962867) (xy -3.17804 0.871448)
    (xy -3.214785 0.795634) (xy -3.240486 0.743299) (xy -3.251307 0.722318) (xy -3.251313 0.722309) (xy -3.272839 0.725486)
    (xy -3.321686 0.740923) (xy -3.385164 0.763837) (xy -3.450579 0.789447) (xy -3.505239 0.812968) (xy -3.536452 0.829619)
    (xy -3.536803 0.82989) (xy -3.550596 0.8614) (xy -3.544702 0.923288) (xy -3.541101 0.940308) (xy -3.532028 1.035831)
    (xy -3.541592 1.140972) (xy -3.566499 1.243837) (xy -3.603452 1.332531) (xy -3.649157 1.39516) (xy -3.671696 1.411668)
    (xy -3.745078 1.435065) (xy -3.806792 1.419439) (xy -3.857858 1.363794) (xy -3.899292 1.267133) (xy -3.925416 1.163436)
    (xy -4.005723 0.815019) (xy -4.102899 0.481466) (xy -4.109492 0.461114) (xy -4.152325 0.311987) (xy -4.171774 0.197708)
    (xy -5.266112 0.197708) (xy -5.13745 0.535868) (xy -4.952247 0.963623) (xy -4.785076 1.315668) (xy -4.701372 1.484308)
    (xy -4.633315 1.616938) (xy -4.578466 1.717101) (xy -4.534383 1.788341) (xy -4.498628 1.834203) (xy -4.468761 1.858229)
    (xy -4.442342 1.863965) (xy -4.416931 1.854954) (xy -4.414738 1.853621) (xy -4.3817 1.841802) (xy -4.335784 1.845492)
    (xy -4.26489 1.86602) (xy -4.247419 1.871996) (xy -4.111386 1.914861) (xy -3.978107 1.946573) (xy -3.83589 1.969002)
    (xy -3.673046 1.984016) (xy -3.490326 1.993055))
   (stroke (width 0) (type solid)) (fill yes) (layer "B.Cu")))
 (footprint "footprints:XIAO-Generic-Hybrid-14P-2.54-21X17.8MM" (layer "B.Cu") (at 133.625 71.54 180)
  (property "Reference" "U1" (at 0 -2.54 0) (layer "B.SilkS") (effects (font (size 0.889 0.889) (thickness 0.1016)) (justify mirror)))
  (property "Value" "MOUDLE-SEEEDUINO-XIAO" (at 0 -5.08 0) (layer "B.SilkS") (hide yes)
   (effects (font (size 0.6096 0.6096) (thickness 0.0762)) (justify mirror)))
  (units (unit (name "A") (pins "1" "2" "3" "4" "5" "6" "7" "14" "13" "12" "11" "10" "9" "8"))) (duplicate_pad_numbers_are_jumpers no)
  (pad "1" thru_hole rect (at -7.625 7.62 180) (size 3.5 1.7) (drill 1 (offset -1 0)) (layers "*.Cu" "*.Mask") (remove_unused_layers no)
   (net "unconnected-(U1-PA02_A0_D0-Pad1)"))
  (pad "2" thru_hole oval (at -7.625 5.08 180) (size 3.6 1.7) (drill 1 (offset -1 0)) (layers "*.Cu" "*.Mask") (remove_unused_layers no)
   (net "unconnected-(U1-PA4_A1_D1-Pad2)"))
  (pad "3" thru_hole oval (at -7.625 2.54 180) (size 3.6 1.7) (drill 1 (offset -1 0)) (layers "*.Cu" "*.Mask") (remove_unused_layers no)
   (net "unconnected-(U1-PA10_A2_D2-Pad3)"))
  (pad "4" thru_hole oval (at -7.625 0 180) (size 3.6 1.7) (drill 1 (offset -1 0)) (layers "*.Cu" "*.Mask") (remove_unused_layers no)
   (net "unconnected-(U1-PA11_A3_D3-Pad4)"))
  (pad "5" thru_hole oval (at -7.625 -2.54 180) (size 3.6 1.7) (drill 1 (offset -1 0)) (layers "*.Cu" "*.Mask") (remove_unused_layers no)
   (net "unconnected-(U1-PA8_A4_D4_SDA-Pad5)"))
  (pad "6" thru_hole oval (at -7.625 -5.08) (size 3.6 1.7) (drill 1 (offset 1 0)) (layers "*.Cu" "*.Mask") (remove_unused_layers no)
   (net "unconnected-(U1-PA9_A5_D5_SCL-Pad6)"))
  (pad "7" thru_hole oval (at -7.625 -7.62 180) (size 3.6 1.7) (drill 1 (offset -1 0)) (layers "*.Cu" "*.Mask") (remove_unused_layers no)
   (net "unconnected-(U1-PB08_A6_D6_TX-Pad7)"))
  (pad "8" thru_hole oval (at 7.625 -7.62 180) (size 3.6 1.7) (drill 1 (offset 1 0)) (layers "*.Cu" "*.Mask") (remove_unused_layers no)
   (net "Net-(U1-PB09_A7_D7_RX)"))
  (pad "9" thru_hole oval (at 7.625 -5.08 180) (size 3.6 1.7) (drill 1 (offset 1 0)) (layers "*.Cu" "*.Mask") (remove_unused_layers no)
   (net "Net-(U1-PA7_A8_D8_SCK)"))
  (pad "10" thru_hole oval (at 7.625 -2.54 180) (size 3.6 1.7) (drill 1 (offset 1 0)) (layers "*.Cu" "*.Mask") (remove_unused_layers no)
   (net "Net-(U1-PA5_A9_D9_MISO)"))
  (pad "11" thru_hole oval (at 7.625 0 180) (size 3.7 1.7) (drill 1 (offset 1 0)) (layers "*.Cu" "*.Mask") (remove_unused_layers no)
   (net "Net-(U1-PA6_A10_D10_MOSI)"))
  (pad "12" thru_hole oval (at 7.625 2.54 180) (size 3.7 1.7) (drill 1 (offset 1 0)) (layers "*.Cu" "*.Mask") (remove_unused_layers no)
   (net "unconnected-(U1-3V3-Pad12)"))
  (pad "13" thru_hole oval (at 7.625 5.08 180) (size 3.7 1.7) (drill 1 (offset 1 0)) (layers "*.Cu" "*.Mask") (remove_unused_layers no)
   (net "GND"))
  (pad "14" thru_hole oval (at 7.625 7.62 180) (size 3.7 1.7) (drill 1 (offset 1 0)) (layers "*.Cu" "*.Mask") (remove_unused_layers no)
   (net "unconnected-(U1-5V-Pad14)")))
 (gr_rect (start 124 61) (end 143 137) (stroke (width 0.05) (type default)) (fill no) (layer "Edge.Cuts"))
 (segment (start 129 85.5) (end 129 80) (width 0.2) (layer "B.Cu") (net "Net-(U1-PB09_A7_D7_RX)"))
 (segment (start 130.254899 85.5) (end 129 85.5) (width 0.2) (layer "B.Cu") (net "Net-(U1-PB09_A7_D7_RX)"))
 (segment (start 129 80) (end 128.16 79.16) (width 0.2) (layer "B.Cu") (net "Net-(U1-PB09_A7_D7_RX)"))
 (segment (start 136.085 107.716598) (end 134.368402 106) (width 0.2) (layer "B.Cu") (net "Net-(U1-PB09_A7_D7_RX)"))
 (segment (start 131.5 106) (end 131.195 105.695) (width 0.2) (layer "B.Cu") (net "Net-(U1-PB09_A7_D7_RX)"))
 (segment (start 131.195 86.440101) (end 130.254899 85.5) (width 0.2) (layer "B.Cu") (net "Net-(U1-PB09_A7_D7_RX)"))
 (segment (start 134.368402 106) (end 131.5 106) (width 0.2) (layer "B.Cu") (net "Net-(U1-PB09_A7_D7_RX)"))
 (segment (start 128.16 79.16) (end 126 79.16) (width 0.2) (layer "B.Cu") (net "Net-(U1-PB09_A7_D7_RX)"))
 (segment (start 131.195 105.695) (end 131.195 86.440101) (width 0.2) (layer "B.Cu") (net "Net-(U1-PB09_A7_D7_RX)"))
 (segment (start 136.085 122.42) (end 136.085 107.716598) (width 0.2) (layer "B.Cu") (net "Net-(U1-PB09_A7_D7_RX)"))
 (segment (start 132 77) (end 131.5 76.5) (width 0.2) (layer "B.Cu") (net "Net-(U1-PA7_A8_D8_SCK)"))
 (segment (start 126.12 76.5) (end 126 76.62) (width 0.2) (layer "B.Cu") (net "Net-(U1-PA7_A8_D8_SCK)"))
 (segment (start 132 87) (end 132 77) (width 0.2) (layer "B.Cu") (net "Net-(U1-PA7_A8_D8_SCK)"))
 (segment (start 136.085 103.42) (end 136.085 88.716598) (width 0.2) (layer "B.Cu") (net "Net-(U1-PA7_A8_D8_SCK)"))
 (segment (start 131.5 76.5) (end 126.12 76.5) (width 0.2) (layer "B.Cu") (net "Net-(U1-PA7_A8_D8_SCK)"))
 (segment (start 136.085 88.716598) (end 134.368402 87) (width 0.2) (layer "B.Cu") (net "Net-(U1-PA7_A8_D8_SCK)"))
 (segment (start 134.368402 87) (end 132 87) (width 0.2) (layer "B.Cu") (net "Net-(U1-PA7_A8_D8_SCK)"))
 (segment (start 135.42 74.08) (end 126 74.08) (width 0.2) (layer "B.Cu") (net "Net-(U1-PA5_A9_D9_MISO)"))
 (segment (start 136.085 74.585) (end 135.5 74) (width 0.2) (layer "B.Cu") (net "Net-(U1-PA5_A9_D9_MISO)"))
 (segment (start 135.5 74) (end 135.42 74.08) (width 0.2) (layer "B.Cu") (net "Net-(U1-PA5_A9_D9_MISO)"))
 (segment (start 136.085 84.42) (end 136.085 74.585) (width 0.2) (layer "B.Cu") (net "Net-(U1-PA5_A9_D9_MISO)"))
 (segment (start 136.085 65.42) (end 136.085 72.415) (width 0.2) (layer "B.Cu") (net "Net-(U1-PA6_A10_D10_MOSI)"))
 (segment (start 135.65 72.85) (end 127.31 72.85) (width 0.2) (layer "B.Cu") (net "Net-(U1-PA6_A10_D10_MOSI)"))
 (segment (start 127.31 72.85) (end 126 71.54) (width 0.2) (layer "B.Cu") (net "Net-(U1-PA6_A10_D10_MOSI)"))
 (segment (start 136.085 72.415) (end 135.65 72.85) (width 0.2) (layer "B.Cu") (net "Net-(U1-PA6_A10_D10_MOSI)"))
 (segment (start 129.735 86.96) (end 129.735 105.96) (width 0.2) (layer "F.Cu") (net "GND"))
 (segment (start 129.735 67.96) (end 129.735 86.96) (width 0.2) (layer "F.Cu") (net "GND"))
 (segment (start 128.235 66.46) (end 129.735 67.96) (width 0.2) (layer "F.Cu") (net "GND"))
 (segment (start 129.735 105.96) (end 129.735 124.96) (width 0.2) (layer "F.Cu") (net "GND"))
 (segment (start 126 66.46) (end 128.235 66.46) (width 0.2) (layer "F.Cu") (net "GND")))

